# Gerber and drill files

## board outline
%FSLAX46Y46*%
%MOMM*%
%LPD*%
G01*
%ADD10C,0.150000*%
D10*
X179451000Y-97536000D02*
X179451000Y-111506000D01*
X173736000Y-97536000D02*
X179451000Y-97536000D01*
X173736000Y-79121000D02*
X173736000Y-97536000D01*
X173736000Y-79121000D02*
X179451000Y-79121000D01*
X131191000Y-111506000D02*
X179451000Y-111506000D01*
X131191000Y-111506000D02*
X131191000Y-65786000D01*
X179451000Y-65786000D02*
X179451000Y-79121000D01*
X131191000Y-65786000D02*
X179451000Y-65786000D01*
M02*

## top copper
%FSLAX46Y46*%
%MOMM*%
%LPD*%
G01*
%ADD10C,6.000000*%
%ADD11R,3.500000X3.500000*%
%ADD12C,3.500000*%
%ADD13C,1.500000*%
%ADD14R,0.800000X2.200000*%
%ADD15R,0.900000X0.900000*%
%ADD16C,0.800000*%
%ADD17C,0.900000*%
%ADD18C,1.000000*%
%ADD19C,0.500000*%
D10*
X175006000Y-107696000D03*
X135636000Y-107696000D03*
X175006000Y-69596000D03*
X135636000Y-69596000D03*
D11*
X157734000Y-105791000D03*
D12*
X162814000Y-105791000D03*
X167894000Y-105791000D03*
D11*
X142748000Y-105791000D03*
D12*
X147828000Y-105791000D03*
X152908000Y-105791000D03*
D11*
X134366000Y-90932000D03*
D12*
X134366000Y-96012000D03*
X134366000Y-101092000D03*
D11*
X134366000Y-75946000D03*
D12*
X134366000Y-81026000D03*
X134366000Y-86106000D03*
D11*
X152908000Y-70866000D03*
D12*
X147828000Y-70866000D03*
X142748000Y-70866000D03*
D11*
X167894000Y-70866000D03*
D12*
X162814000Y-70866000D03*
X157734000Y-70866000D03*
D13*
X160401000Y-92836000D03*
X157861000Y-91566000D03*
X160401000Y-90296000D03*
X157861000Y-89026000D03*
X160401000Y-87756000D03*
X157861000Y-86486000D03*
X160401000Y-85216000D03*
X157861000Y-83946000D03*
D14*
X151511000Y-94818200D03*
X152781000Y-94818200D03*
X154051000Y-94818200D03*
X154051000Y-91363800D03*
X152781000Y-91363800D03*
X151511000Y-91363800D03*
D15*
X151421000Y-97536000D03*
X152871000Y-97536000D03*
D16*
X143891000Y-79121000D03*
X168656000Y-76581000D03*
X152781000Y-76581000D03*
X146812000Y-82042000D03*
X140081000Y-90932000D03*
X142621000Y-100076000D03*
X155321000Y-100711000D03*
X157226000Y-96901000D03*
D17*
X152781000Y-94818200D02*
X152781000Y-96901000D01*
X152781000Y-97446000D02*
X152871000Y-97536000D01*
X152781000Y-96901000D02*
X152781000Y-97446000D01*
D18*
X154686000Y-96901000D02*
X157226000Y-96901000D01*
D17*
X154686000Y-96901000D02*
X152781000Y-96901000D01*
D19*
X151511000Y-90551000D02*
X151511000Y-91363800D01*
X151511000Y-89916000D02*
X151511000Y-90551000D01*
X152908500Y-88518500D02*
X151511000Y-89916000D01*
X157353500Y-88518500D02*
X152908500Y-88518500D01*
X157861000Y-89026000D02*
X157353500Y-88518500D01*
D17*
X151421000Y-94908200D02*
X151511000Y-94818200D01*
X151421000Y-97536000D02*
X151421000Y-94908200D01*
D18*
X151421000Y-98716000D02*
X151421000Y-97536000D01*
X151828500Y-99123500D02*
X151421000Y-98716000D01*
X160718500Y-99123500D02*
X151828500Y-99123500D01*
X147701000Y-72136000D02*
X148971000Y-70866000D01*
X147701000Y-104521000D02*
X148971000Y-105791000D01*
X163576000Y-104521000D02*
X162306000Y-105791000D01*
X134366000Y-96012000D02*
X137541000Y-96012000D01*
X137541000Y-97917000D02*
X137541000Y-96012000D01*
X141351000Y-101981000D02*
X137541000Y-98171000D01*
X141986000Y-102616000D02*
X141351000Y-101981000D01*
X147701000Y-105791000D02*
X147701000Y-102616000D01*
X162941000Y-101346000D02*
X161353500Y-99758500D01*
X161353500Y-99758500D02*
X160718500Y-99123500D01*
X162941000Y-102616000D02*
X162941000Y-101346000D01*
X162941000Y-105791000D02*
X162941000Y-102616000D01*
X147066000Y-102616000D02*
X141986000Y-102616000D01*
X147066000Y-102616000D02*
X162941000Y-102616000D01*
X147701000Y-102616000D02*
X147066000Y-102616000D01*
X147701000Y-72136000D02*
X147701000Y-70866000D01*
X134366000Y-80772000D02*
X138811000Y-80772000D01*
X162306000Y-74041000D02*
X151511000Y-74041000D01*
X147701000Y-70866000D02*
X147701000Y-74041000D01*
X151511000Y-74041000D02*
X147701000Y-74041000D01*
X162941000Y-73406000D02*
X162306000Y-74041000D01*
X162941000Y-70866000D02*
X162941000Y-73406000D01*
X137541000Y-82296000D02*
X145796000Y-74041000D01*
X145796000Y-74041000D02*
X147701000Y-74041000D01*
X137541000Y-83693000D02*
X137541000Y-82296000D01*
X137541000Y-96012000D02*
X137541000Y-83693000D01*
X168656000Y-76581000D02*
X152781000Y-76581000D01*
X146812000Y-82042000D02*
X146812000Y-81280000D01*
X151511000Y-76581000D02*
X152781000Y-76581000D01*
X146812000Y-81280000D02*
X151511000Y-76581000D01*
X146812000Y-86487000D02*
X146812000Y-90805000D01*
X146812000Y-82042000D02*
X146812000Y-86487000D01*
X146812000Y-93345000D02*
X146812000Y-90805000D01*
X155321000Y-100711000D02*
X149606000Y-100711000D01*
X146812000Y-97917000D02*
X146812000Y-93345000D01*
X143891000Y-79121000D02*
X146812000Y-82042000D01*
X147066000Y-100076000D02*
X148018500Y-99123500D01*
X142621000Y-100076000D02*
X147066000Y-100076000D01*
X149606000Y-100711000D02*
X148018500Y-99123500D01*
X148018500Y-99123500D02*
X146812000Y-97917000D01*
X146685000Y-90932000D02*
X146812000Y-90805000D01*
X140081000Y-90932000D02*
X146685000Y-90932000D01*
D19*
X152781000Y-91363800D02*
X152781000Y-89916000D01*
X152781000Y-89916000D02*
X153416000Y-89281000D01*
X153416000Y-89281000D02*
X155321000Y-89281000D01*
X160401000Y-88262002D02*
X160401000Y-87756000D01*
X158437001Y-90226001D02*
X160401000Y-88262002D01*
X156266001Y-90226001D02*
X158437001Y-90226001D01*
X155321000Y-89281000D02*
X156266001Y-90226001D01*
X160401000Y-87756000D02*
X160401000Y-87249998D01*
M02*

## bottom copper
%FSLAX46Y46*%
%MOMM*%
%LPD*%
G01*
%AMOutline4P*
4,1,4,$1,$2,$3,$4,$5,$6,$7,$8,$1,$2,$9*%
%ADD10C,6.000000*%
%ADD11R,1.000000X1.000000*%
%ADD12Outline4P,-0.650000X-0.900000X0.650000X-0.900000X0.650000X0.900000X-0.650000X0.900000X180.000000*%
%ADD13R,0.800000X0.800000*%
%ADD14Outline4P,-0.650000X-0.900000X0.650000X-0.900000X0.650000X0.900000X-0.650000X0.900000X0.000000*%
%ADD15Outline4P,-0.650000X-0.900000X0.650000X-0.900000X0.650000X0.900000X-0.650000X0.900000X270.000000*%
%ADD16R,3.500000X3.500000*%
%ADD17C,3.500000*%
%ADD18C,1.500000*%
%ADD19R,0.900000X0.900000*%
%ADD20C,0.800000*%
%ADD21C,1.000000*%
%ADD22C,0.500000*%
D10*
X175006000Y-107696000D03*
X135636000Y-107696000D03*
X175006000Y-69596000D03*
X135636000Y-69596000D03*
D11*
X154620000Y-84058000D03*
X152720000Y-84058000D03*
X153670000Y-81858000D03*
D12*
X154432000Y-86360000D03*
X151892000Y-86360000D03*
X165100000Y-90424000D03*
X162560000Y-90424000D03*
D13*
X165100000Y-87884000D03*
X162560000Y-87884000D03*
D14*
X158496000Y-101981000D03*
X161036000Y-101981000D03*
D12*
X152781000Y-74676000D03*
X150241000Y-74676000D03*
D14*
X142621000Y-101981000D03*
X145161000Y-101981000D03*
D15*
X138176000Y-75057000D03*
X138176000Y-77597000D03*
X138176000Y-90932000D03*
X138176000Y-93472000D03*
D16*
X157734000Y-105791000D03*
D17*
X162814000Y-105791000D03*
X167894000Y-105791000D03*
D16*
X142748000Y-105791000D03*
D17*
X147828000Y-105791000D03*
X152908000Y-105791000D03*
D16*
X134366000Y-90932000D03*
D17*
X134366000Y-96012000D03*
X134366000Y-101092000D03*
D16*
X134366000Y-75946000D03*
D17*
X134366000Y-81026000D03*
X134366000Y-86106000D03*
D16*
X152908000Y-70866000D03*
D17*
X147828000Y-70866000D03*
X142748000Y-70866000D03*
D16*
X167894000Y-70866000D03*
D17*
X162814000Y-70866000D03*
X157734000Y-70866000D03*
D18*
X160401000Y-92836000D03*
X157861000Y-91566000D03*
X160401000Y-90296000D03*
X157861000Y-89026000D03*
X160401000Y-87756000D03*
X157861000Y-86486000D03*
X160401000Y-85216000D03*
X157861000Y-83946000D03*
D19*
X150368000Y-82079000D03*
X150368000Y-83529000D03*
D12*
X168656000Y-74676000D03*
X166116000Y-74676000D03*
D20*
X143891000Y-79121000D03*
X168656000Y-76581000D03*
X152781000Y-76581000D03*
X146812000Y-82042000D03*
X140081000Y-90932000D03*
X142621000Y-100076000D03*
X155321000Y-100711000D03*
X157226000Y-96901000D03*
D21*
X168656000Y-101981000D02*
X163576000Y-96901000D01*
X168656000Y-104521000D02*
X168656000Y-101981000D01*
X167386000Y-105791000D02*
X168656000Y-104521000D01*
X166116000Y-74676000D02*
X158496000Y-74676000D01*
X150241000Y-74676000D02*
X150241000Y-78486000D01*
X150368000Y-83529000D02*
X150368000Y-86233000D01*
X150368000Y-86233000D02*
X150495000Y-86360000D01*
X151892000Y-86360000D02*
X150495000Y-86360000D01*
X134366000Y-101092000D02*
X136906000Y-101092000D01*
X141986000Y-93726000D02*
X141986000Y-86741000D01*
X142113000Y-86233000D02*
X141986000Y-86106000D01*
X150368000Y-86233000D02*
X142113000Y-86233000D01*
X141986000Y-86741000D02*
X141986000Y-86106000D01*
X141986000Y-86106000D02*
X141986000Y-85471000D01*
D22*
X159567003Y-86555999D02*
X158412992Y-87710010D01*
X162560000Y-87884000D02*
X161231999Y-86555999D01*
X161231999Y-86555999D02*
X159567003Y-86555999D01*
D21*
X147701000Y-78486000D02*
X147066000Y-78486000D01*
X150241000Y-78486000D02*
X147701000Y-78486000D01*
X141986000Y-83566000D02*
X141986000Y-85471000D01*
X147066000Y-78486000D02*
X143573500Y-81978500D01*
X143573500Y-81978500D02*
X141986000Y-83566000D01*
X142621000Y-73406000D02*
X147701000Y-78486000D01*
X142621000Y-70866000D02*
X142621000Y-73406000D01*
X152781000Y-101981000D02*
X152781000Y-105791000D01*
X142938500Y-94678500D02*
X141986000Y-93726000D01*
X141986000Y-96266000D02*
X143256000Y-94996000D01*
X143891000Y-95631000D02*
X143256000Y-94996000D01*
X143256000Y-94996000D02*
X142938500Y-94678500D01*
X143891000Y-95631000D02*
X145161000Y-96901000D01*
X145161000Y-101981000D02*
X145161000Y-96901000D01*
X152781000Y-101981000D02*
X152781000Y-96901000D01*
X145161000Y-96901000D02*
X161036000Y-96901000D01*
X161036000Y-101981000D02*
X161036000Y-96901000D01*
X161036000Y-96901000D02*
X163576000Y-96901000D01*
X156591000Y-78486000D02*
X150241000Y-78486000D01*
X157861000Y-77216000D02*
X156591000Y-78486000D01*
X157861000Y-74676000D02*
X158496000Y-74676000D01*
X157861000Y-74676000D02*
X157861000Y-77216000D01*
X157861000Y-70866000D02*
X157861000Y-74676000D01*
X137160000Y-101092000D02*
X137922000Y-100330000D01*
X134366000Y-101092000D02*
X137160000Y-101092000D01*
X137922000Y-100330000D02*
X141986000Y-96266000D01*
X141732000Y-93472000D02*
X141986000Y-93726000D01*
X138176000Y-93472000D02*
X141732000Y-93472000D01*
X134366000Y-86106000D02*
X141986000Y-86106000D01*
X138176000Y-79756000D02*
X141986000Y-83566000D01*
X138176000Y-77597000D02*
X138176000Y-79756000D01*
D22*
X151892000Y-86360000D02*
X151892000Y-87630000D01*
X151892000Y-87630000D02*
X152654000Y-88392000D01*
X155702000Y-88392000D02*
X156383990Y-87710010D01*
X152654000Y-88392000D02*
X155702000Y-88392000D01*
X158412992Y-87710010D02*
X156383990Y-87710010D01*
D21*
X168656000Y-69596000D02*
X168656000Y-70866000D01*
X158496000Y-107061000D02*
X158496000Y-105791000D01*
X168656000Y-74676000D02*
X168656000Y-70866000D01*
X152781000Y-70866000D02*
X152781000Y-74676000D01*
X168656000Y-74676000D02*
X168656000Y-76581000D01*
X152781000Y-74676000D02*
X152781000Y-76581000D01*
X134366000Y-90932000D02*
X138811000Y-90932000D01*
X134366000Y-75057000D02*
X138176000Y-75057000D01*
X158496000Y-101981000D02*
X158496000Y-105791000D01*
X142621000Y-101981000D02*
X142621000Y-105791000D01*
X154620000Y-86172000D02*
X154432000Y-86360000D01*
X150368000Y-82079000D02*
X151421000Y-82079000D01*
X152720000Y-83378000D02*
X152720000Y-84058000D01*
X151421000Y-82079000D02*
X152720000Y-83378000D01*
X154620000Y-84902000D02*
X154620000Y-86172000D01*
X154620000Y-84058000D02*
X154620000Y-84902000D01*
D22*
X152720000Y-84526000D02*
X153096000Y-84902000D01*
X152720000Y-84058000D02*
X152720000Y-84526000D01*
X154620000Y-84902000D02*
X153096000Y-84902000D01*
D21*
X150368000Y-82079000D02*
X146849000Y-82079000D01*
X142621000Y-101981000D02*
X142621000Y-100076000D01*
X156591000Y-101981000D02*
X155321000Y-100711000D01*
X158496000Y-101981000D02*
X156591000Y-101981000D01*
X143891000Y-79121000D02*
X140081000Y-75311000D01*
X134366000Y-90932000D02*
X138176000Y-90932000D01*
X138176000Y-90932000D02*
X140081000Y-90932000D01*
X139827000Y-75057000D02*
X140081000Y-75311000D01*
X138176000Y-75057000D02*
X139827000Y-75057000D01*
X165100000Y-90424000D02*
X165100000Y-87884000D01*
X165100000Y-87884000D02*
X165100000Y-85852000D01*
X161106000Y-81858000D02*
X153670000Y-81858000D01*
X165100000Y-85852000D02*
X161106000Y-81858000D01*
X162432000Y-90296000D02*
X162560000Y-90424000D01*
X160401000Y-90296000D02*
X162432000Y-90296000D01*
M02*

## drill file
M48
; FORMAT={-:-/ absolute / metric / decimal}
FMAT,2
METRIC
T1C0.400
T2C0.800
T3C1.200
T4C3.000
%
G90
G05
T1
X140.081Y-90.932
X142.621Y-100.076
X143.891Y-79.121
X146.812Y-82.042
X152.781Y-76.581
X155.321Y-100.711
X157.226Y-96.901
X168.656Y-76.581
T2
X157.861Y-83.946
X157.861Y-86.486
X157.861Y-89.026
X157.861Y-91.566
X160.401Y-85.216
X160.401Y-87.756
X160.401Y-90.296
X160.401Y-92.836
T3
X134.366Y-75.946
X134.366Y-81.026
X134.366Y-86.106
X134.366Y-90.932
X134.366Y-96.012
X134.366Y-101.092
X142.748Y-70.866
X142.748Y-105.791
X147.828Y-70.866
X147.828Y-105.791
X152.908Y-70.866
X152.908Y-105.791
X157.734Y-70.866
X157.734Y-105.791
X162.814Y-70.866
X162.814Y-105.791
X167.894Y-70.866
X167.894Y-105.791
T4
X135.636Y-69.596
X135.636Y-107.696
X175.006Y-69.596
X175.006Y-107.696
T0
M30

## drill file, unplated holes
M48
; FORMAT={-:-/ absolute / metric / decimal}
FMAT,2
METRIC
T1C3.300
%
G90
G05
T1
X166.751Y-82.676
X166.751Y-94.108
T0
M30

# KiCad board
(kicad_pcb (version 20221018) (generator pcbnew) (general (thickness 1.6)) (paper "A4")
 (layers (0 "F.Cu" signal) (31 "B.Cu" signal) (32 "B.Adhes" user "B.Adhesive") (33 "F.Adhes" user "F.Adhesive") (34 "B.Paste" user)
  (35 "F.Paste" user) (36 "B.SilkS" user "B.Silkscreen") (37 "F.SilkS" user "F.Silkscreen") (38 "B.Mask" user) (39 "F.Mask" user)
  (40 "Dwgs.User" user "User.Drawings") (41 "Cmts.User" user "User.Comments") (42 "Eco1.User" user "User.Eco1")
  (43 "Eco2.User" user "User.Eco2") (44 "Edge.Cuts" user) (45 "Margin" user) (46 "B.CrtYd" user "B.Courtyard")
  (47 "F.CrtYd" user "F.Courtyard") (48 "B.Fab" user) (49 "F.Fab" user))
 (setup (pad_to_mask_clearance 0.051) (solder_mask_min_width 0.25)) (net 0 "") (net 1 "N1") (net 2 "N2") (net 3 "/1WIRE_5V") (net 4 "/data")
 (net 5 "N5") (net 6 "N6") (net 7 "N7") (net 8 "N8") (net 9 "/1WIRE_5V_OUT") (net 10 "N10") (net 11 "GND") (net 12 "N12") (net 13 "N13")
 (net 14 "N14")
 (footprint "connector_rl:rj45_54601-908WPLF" (layer "F.Cu") (at 166.751 88.392 90)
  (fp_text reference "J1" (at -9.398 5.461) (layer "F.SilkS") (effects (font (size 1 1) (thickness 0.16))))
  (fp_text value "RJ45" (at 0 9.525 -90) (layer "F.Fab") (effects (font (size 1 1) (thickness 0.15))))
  (pad "" np_thru_hole circle (at -5.716 0 90) (size 3.3 3.3) (drill 3.3) (layers "*.Cu" "*.SilkS" "*.Mask"))
  (pad "" np_thru_hole circle (at 5.716 0 90) (size 3.3 3.3) (drill 3.3) (layers "*.Cu" "*.SilkS" "*.Mask"))
  (pad "1" thru_hole circle (at -4.444 -6.35 90) (size 1.5 1.5) (drill 0.8) (layers "*.Cu" "*.Mask") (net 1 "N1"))
  (pad "2" thru_hole circle (at -3.174 -8.89 90) (size 1.5 1.5) (drill 0.8) (layers "*.Cu" "*.Mask") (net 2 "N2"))
  (pad "3" thru_hole circle (at -1.904 -6.35 90) (size 1.5 1.5) (drill 0.8) (layers "*.Cu" "*.Mask") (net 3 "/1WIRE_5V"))
  (pad "4" thru_hole circle (at -0.634 -8.89 90) (size 1.5 1.5) (drill 0.8) (layers "*.Cu" "*.Mask") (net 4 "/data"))
  (pad "5" thru_hole circle (at 0.636 -6.35 90) (size 1.5 1.5) (drill 0.8) (layers "*.Cu" "*.Mask") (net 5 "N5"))
  (pad "6" thru_hole circle (at 1.906 -8.89 270) (size 1.5 1.5) (drill 0.8) (layers "*.Cu" "*.Mask") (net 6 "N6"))
  (pad "7" thru_hole circle (at 3.176 -6.35 90) (size 1.5 1.5) (drill 0.8) (layers "*.Cu" "*.Mask") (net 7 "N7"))
  (pad "8" thru_hole circle (at 4.446 -8.89 90) (size 1.5 1.5) (drill 0.8) (layers "*.Cu" "*.Mask") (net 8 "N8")))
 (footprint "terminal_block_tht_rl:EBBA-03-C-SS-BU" (layer "F.Cu") (at 162.814 70.866 180)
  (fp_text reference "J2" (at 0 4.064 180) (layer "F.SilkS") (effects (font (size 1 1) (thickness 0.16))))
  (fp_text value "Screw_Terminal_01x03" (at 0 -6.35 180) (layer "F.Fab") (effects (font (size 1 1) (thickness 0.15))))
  (pad "1" thru_hole rect (at -5.08 0) (size 3.5 3.5) (drill 1.2) (layers "*.Cu" "*.Mask") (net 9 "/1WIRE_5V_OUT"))
  (pad "2" thru_hole circle (at 0 0) (size 3.5 3.5) (drill 1.2) (layers "*.Cu" "*.Mask") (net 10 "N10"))
  (pad "3" thru_hole circle (at 5.08 0) (size 3.5 3.5) (drill 1.2) (layers "*.Cu" "*.Mask") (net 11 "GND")))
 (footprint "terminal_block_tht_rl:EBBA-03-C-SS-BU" (layer "F.Cu") (at 134.366 81.026 -90)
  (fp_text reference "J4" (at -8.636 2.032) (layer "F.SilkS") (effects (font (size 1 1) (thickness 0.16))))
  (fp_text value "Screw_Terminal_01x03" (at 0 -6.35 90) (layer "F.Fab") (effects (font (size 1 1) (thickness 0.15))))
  (pad "1" thru_hole rect (at -5.08 0 90) (size 3.5 3.5) (drill 1.2) (layers "*.Cu" "*.Mask") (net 9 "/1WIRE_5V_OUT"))
  (pad "2" thru_hole circle (at 0 0 90) (size 3.5 3.5) (drill 1.2) (layers "*.Cu" "*.Mask") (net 10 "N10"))
  (pad "3" thru_hole circle (at 5.08 0 90) (size 3.5 3.5) (drill 1.2) (layers "*.Cu" "*.Mask") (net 11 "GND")))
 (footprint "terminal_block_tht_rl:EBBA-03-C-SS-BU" (layer "F.Cu") (at 134.366 96.012 -90)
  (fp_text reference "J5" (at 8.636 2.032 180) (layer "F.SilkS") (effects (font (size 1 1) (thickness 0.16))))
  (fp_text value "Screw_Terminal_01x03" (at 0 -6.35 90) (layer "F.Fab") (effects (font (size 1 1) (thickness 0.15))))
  (pad "1" thru_hole rect (at -5.08 0 90) (size 3.5 3.5) (drill 1.2) (layers "*.Cu" "*.Mask") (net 9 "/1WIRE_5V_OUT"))
  (pad "2" thru_hole circle (at 0 0 90) (size 3.5 3.5) (drill 1.2) (layers "*.Cu" "*.Mask") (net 10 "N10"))
  (pad "3" thru_hole circle (at 5.08 0 90) (size 3.5 3.5) (drill 1.2) (layers "*.Cu" "*.Mask") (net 11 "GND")))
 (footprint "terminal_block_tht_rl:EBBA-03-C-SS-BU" (layer "F.Cu") (at 147.828 70.866 180)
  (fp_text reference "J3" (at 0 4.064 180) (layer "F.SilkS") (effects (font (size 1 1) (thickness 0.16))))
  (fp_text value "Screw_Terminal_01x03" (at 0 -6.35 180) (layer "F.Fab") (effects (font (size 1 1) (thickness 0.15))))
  (pad "1" thru_hole rect (at -5.08 0) (size 3.5 3.5) (drill 1.2) (layers "*.Cu" "*.Mask") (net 9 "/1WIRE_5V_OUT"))
  (pad "2" thru_hole circle (at 0 0) (size 3.5 3.5) (drill 1.2) (layers "*.Cu" "*.Mask") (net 10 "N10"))
  (pad "3" thru_hole circle (at 5.08 0) (size 3.5 3.5) (drill 1.2) (layers "*.Cu" "*.Mask") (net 11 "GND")))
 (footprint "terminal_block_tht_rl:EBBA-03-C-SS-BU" (layer "F.Cu") (at 147.828 105.791)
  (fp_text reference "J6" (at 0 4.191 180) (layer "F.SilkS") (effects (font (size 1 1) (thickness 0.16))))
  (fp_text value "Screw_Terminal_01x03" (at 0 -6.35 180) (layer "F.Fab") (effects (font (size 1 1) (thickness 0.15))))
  (pad "1" thru_hole rect (at -5.08 0 180) (size 3.5 3.5) (drill 1.2) (layers "*.Cu" "*.Mask") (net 9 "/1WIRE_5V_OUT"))
  (pad "2" thru_hole circle (at 0 0 180) (size 3.5 3.5) (drill 1.2) (layers "*.Cu" "*.Mask") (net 10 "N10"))
  (pad "3" thru_hole circle (at 5.08 0 180) (size 3.5 3.5) (drill 1.2) (layers "*.Cu" "*.Mask") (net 11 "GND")))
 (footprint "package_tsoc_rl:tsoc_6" (layer "F.Cu") (at 152.781 93.091 90)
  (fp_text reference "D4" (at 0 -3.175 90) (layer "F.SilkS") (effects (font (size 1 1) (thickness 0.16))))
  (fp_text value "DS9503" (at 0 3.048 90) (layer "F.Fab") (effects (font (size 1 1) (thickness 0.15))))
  (pad "1" smd rect (at -1.7272 -1.27 90) (size 2.2 0.8) (layers "F.Cu" "F.Paste" "F.Mask") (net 10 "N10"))
  (pad "2" smd rect (at -1.7272 0 90) (size 2.2 0.8) (layers "F.Cu" "F.Paste" "F.Mask") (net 11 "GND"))
  (pad "3" smd rect (at -1.7272 1.27 90) (size 2.2 0.8) (layers "F.Cu" "F.Paste" "F.Mask") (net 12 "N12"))
  (pad "4" smd rect (at 1.7272 1.27 90) (size 2.2 0.8) (layers "F.Cu" "F.Paste" "F.Mask") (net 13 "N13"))
  (pad "5" smd rect (at 1.7272 0 90) (size 2.2 0.8) (layers "F.Cu" "F.Paste" "F.Mask") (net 5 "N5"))
  (pad "6" smd rect (at 1.7272 -1.27 90) (size 2.2 0.8) (layers "F.Cu" "F.Paste" "F.Mask") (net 4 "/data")))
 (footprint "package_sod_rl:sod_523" (layer "F.Cu") (at 152.146 97.536)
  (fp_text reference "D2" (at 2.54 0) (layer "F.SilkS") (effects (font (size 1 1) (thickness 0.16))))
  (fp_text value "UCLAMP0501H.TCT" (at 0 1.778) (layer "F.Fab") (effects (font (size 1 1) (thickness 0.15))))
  (pad "1" smd rect (at -0.725 0) (size 0.9 0.9) (layers "F.Cu" "F.Paste" "F.Mask") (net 10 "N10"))
  (pad "2" smd rect (at 0.725 0) (size 0.9 0.9) (layers "F.Cu" "F.Paste" "F.Mask") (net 11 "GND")))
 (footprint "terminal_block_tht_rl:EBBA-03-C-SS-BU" (layer "F.Cu") (at 162.814 105.791)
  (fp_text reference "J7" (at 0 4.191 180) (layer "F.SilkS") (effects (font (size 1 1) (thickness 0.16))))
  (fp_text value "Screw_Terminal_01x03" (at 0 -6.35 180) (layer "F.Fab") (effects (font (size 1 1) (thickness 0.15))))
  (pad "1" thru_hole rect (at -5.08 0 180) (size 3.5 3.5) (drill 1.2) (layers "*.Cu" "*.Mask") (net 9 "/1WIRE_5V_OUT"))
  (pad "2" thru_hole circle (at 0 0 180) (size 3.5 3.5) (drill 1.2) (layers "*.Cu" "*.Mask") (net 10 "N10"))
  (pad "3" thru_hole circle (at 5.08 0 180) (size 3.5 3.5) (drill 1.2) (layers "*.Cu" "*.Mask") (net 11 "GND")))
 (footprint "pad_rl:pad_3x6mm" (layer "F.Cu") (at 135.636 69.596)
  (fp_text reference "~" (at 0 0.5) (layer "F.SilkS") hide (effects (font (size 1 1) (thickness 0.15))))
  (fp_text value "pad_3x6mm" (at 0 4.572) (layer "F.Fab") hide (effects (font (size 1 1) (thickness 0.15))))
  (pad "~" thru_hole circle (at 0 0) (size 6 6) (drill 3) (layers "*.Cu" "*.Mask")))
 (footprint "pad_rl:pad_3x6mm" (layer "F.Cu") (at 175.006 69.596)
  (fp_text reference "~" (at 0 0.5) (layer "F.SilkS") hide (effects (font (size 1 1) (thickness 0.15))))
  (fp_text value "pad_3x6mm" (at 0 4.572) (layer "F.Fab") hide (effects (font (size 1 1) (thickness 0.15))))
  (pad "~" thru_hole circle (at 0 0) (size 6 6) (drill 3) (layers "*.Cu" "*.Mask")))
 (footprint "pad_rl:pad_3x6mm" (layer "F.Cu") (at 135.636 107.696)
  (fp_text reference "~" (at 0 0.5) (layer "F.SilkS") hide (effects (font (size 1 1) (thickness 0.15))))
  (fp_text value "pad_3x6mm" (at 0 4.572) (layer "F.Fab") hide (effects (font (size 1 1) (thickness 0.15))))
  (pad "~" thru_hole circle (at 0 0) (size 6 6) (drill 3) (layers "*.Cu" "*.Mask")))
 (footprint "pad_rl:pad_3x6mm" (layer "F.Cu") (at 175.006 107.696)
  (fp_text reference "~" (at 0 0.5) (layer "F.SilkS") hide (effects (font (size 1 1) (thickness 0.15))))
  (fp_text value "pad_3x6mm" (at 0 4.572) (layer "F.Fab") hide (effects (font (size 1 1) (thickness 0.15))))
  (pad "~" thru_hole circle (at 0 0) (size 6 6) (drill 3) (layers "*.Cu" "*.Mask")))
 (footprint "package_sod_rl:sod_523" (layer "B.Cu") (at 150.368 82.804 -90)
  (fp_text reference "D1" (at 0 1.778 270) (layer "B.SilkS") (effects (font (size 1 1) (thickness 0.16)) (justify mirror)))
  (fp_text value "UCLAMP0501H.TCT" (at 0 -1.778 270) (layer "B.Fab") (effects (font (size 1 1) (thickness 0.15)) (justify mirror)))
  (pad "1" smd rect (at -0.725 0 270) (size 0.9 0.9) (layers "B.Cu" "B.Paste" "B.Mask") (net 9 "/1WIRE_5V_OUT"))
  (pad "2" smd rect (at 0.725 0 270) (size 0.9 0.9) (layers "B.Cu" "B.Paste" "B.Mask") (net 11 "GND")))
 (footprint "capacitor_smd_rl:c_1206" (layer "B.Cu") (at 167.386 74.676 180)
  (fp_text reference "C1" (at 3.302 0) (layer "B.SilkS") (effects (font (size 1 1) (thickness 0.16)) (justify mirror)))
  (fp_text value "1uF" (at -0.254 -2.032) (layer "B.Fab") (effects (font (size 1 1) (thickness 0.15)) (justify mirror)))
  (pad "1" smd trapezoid (at -1.27 0 180) (size 1.3 1.8) (layers "B.Cu" "B.Paste" "B.Mask") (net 9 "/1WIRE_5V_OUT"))
  (pad "2" smd trapezoid (at 1.27 0 180) (size 1.3 1.8) (layers "B.Cu" "B.Paste" "B.Mask") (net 11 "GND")))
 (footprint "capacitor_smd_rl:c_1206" (layer "B.Cu") (at 138.176 92.202 -90)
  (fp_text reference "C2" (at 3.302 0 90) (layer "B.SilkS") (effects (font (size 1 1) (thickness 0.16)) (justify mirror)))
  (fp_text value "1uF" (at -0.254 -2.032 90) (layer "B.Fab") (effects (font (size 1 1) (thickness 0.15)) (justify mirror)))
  (pad "1" smd trapezoid (at -1.27 0 270) (size 1.3 1.8) (layers "B.Cu" "B.Paste" "B.Mask") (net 9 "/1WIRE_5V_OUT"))
  (pad "2" smd trapezoid (at 1.27 0 270) (size 1.3 1.8) (layers "B.Cu" "B.Paste" "B.Mask") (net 11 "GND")))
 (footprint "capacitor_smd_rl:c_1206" (layer "B.Cu") (at 151.511 74.676 180)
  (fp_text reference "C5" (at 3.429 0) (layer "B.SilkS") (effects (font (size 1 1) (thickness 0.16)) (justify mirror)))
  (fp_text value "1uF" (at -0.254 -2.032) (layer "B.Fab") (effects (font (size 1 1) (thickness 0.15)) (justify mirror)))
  (pad "1" smd trapezoid (at -1.27 0 180) (size 1.3 1.8) (layers "B.Cu" "B.Paste" "B.Mask") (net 9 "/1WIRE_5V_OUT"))
  (pad "2" smd trapezoid (at 1.27 0 180) (size 1.3 1.8) (layers "B.Cu" "B.Paste" "B.Mask") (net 11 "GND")))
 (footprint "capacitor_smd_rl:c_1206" (layer "B.Cu") (at 143.891 101.981)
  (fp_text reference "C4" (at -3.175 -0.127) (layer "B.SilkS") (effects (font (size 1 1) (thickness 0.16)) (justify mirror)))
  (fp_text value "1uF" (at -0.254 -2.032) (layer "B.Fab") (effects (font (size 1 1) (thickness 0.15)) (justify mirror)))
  (pad "1" smd trapezoid (at -1.27 0) (size 1.3 1.8) (layers "B.Cu" "B.Paste" "B.Mask") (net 9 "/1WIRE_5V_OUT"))
  (pad "2" smd trapezoid (at 1.27 0) (size 1.3 1.8) (layers "B.Cu" "B.Paste" "B.Mask") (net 11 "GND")))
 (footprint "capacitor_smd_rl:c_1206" (layer "B.Cu") (at 159.766 101.981)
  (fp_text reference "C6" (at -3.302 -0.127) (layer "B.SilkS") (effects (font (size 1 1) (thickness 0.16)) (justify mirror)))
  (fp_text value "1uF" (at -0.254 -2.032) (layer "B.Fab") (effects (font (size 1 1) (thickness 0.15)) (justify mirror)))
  (pad "1" smd trapezoid (at -1.27 0) (size 1.3 1.8) (layers "B.Cu" "B.Paste" "B.Mask") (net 9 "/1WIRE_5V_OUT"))
  (pad "2" smd trapezoid (at 1.27 0) (size 1.3 1.8) (layers "B.Cu" "B.Paste" "B.Mask") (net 11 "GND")))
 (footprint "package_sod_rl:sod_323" (layer "B.Cu") (at 163.83 87.884 180)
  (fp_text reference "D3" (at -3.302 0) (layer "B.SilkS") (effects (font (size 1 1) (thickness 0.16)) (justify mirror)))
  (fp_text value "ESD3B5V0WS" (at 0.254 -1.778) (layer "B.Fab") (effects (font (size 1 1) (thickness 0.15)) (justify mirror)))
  (pad "1" smd rect (at -1.27 0 180) (size 0.8 0.8) (layers "B.Cu" "B.Paste" "B.Mask") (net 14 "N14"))
  (pad "2" smd rect (at 1.27 0 180) (size 0.8 0.8) (layers "B.Cu" "B.Paste" "B.Mask") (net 11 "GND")))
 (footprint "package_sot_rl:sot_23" (layer "B.Cu") (at 153.67 83.058 90)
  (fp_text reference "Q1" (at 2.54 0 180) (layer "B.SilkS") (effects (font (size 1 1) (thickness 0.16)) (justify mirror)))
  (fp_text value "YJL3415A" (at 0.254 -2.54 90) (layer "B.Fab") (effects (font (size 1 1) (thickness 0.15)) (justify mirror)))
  (pad "1" smd rect (at -1 0.95 90) (size 1 1) (layers "B.Cu" "B.Paste" "B.Mask") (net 9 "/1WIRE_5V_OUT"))
  (pad "2" smd rect (at -1 -0.95 90) (size 1 1) (layers "B.Cu" "B.Paste" "B.Mask") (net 9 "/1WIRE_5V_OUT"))
  (pad "3" smd rect (at 1.2 0 90) (size 1 1) (layers "B.Cu" "B.Paste" "B.Mask") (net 14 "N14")))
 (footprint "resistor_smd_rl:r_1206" (layer "B.Cu") (at 163.83 90.424 180)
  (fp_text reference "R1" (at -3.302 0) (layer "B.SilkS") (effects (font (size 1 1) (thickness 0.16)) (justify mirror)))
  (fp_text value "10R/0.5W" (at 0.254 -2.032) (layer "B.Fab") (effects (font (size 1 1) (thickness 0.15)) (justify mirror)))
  (pad "1" smd trapezoid (at -1.27 0 180) (size 1.3 1.8) (layers "B.Cu" "B.Paste" "B.Mask") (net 14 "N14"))
  (pad "2" smd trapezoid (at 1.27 0 180) (size 1.3 1.8) (layers "B.Cu" "B.Paste" "B.Mask") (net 3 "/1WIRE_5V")))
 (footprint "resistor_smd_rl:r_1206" (layer "B.Cu") (at 153.162 86.36 180)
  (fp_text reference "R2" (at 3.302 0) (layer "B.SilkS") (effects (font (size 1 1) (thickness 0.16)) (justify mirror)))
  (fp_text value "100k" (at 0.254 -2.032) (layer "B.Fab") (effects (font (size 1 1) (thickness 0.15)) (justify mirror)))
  (pad "1" smd trapezoid (at -1.27 0 180) (size 1.3 1.8) (layers "B.Cu" "B.Paste" "B.Mask") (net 9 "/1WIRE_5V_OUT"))
  (pad "2" smd trapezoid (at 1.27 0 180) (size 1.3 1.8) (layers "B.Cu" "B.Paste" "B.Mask") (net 11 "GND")))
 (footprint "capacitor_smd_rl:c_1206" (layer "B.Cu") (at 138.176 76.327 -90)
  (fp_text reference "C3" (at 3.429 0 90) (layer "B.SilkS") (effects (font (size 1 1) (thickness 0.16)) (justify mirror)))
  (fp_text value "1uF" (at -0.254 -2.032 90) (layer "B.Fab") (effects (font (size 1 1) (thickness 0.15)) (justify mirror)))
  (pad "1" smd trapezoid (at -1.27 0 270) (size 1.3 1.8) (layers "B.Cu" "B.Paste" "B.Mask") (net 9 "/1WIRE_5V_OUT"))
  (pad "2" smd trapezoid (at 1.27 0 270) (size 1.3 1.8) (layers "B.Cu" "B.Paste" "B.Mask") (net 11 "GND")))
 (gr_line (start 131.191 111.506) (end 131.191 65.786) (stroke (width 0.15) (type solid)) (layer "Edge.Cuts"))
 (gr_line (start 179.451 65.786) (end 179.451 79.121) (stroke (width 0.15) (type solid)) (layer "Edge.Cuts"))
 (gr_line (start 131.191 111.506) (end 179.451 111.506) (stroke (width 0.15) (type solid)) (layer "Edge.Cuts"))
 (gr_line (start 173.736 79.121) (end 179.451 79.121) (stroke (width 0.15) (type solid)) (layer "Edge.Cuts"))
 (gr_line (start 173.736 79.121) (end 173.736 97.536) (stroke (width 0.15) (type solid)) (layer "Edge.Cuts"))
 (gr_line (start 173.736 97.536) (end 179.451 97.536) (stroke (width 0.15) (type solid)) (layer "Edge.Cuts"))
 (gr_line (start 179.451 97.536) (end 179.451 111.506) (stroke (width 0.15) (type solid)) (layer "Edge.Cuts"))
 (gr_line (start 131.191 65.786) (end 179.451 65.786) (stroke (width 0.15) (type solid)) (layer "Edge.Cuts"))
 (segment (start 152.781 94.8182) (end 152.781 96.901) (width 0.9) (layer "F.Cu") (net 11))
 (segment (start 154.686 96.901) (end 157.226 96.901) (width 1) (layer "F.Cu") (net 11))
 (segment (start 152.781 97.446) (end 152.871 97.536) (width 0.9) (layer "F.Cu") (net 11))
 (segment (start 154.686 96.901) (end 152.781 96.901) (width 0.9) (layer "F.Cu") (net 11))
 (segment (start 152.781 96.901) (end 152.781 97.446) (width 0.9) (layer "F.Cu") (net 11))
 (via (at 157.226 96.901) (size 0.8) (drill 0.4) (layers "F.Cu" "B.Cu") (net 11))
 (segment (start 141.986 83.566) (end 141.986 85.471) (width 1) (layer "B.Cu") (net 11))
 (segment (start 142.621 73.406) (end 147.701 78.486) (width 1) (layer "B.Cu") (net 11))
 (segment (start 138.176 79.756) (end 141.986 83.566) (width 1) (layer "B.Cu") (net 11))
 (segment (start 141.986 93.726) (end 141.986 86.741) (width 1) (layer "B.Cu") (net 11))
 (segment (start 150.241 74.676) (end 150.241 78.486) (width 1) (layer "B.Cu") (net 11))
 (segment (start 151.892 86.36) (end 150.495 86.36) (width 1) (layer "B.Cu") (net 11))
 (segment (start 137.922 100.33) (end 141.986 96.266) (width 1) (layer "B.Cu") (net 11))
 (segment (start 150.368 86.233) (end 150.495 86.36) (width 1) (layer "B.Cu") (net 11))
 (segment (start 168.656 104.521) (end 168.656 101.981) (width 1) (layer "B.Cu") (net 11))
 (segment (start 143.891 95.631) (end 143.256 94.996) (width 1) (layer "B.Cu") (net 11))
 (segment (start 137.16 101.092) (end 137.922 100.33) (width 1) (layer "B.Cu") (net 11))
 (segment (start 134.366 86.106) (end 141.986 86.106) (width 1) (layer "B.Cu") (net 11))
 (segment (start 141.732 93.472) (end 141.986 93.726) (width 1) (layer "B.Cu") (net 11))
 (segment (start 167.386 105.791) (end 168.656 104.521) (width 1) (layer "B.Cu") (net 11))
 (segment (start 155.702 88.392) (end 156.38399 87.71001) (width 0.5) (layer "B.Cu") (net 11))
 (segment (start 147.701 78.486) (end 147.066 78.486) (width 1) (layer "B.Cu") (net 11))
 (segment (start 161.036 101.981) (end 161.036 96.901) (width 1) (layer "B.Cu") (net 11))
 (segment (start 168.656 101.981) (end 163.576 96.901) (width 1) (layer "B.Cu") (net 11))
 (segment (start 150.368 83.529) (end 150.368 86.233) (width 1) (layer "B.Cu") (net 11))
 (segment (start 158.412992 87.71001) (end 156.38399 87.71001) (width 0.5) (layer "B.Cu") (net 11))
 (segment (start 145.161 96.901) (end 161.036 96.901) (width 1) (layer "B.Cu") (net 11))
 (segment (start 145.161 101.981) (end 145.161 96.901) (width 1) (layer "B.Cu") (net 11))
 (segment (start 161.231999 86.555999) (end 159.567003 86.555999) (width 0.5) (layer "B.Cu") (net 11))
 (segment (start 159.567003 86.555999) (end 158.412992 87.71001) (width 0.5) (layer "B.Cu") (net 11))
 (segment (start 152.781 101.981) (end 152.781 105.791) (width 1) (layer "B.Cu") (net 11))
 (segment (start 150.368 86.233) (end 142.113 86.233) (width 1) (layer "B.Cu") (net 11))
 (segment (start 166.116 74.676) (end 158.496 74.676) (width 1) (layer "B.Cu") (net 11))
 (segment (start 152.654 88.392) (end 155.702 88.392) (width 0.5) (layer "B.Cu") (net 11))
 (segment (start 142.9385 94.6785) (end 141.986 93.726) (width 1) (layer "B.Cu") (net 11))
 (segment (start 162.56 87.884) (end 161.231999 86.555999) (width 0.5) (layer "B.Cu") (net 11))
 (segment (start 138.176 93.472) (end 141.732 93.472) (width 1) (layer "B.Cu") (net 11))
 (segment (start 152.781 101.981) (end 152.781 96.901) (width 1) (layer "B.Cu") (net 11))
 (segment (start 143.891 95.631) (end 145.161 96.901) (width 1) (layer "B.Cu") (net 11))
 (segment (start 143.256 94.996) (end 142.9385 94.6785) (width 1) (layer "B.Cu") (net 11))
 (segment (start 151.892 87.63) (end 152.654 88.392) (width 0.5) (layer "B.Cu") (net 11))
 (segment (start 142.113 86.233) (end 141.986 86.106) (width 1) (layer "B.Cu") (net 11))
 (segment (start 151.892 86.36) (end 151.892 87.63) (width 0.5) (layer "B.Cu") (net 11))
 (segment (start 134.366 101.092) (end 136.906 101.092) (width 1) (layer "B.Cu") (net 11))
 (segment (start 157.861 74.676) (end 157.861 77.216) (width 1) (layer "B.Cu") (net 11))
 (segment (start 143.5735 81.9785) (end 141.986 83.566) (width 1) (layer "B.Cu") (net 11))
 (segment (start 142.621 70.866) (end 142.621 73.406) (width 1) (layer "B.Cu") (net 11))
 (segment (start 157.861 74.676) (end 158.496 74.676) (width 1) (layer "B.Cu") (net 11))
 (segment (start 134.366 101.092) (end 137.16 101.092) (width 1) (layer "B.Cu") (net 11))
 (segment (start 147.066 78.486) (end 143.5735 81.9785) (width 1) (layer "B.Cu") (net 11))
 (segment (start 138.176 77.597) (end 138.176 79.756) (width 1) (layer "B.Cu") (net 11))
 (segment (start 141.986 96.266) (end 143.256 94.996) (width 1) (layer "B.Cu") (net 11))
 (segment (start 157.861 77.216) (end 156.591 78.486) (width 1) (layer "B.Cu") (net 11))
 (segment (start 156.591 78.486) (end 150.241 78.486) (width 1) (layer "B.Cu") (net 11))
 (segment (start 150.241 78.486) (end 147.701 78.486) (width 1) (layer "B.Cu") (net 11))
 (segment (start 161.036 96.901) (end 163.576 96.901) (width 1) (layer "B.Cu") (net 11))
 (segment (start 157.861 70.866) (end 157.861 74.676) (width 1) (layer "B.Cu") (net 11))
 (segment (start 141.986 86.106) (end 141.986 85.471) (width 1) (layer "B.Cu") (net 11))
 (segment (start 141.986 86.741) (end 141.986 86.106) (width 1) (layer "B.Cu") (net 11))
 (segment (start 152.9085 88.5185) (end 151.511 89.916) (width 0.5) (layer "F.Cu") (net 4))
 (segment (start 151.511 89.916) (end 151.511 90.551) (width 0.5) (layer "F.Cu") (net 4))
 (segment (start 151.511 90.551) (end 151.511 91.3638) (width 0.5) (layer "F.Cu") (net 4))
 (segment (start 157.3535 88.5185) (end 152.9085 88.5185) (width 0.5) (layer "F.Cu") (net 4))
 (segment (start 157.861 89.026) (end 157.3535 88.5185) (width 0.5) (layer "F.Cu") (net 4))
 (segment (start 134.366 96.012) (end 137.541 96.012) (width 1) (layer "F.Cu") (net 10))
 (segment (start 137.541 96.012) (end 137.541 83.693) (width 1) (layer "F.Cu") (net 10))
 (segment (start 141.351 101.981) (end 137.541 98.171) (width 1) (layer "F.Cu") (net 10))
 (segment (start 162.941 101.346) (end 161.3535 99.7585) (width 1) (layer "F.Cu") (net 10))
 (segment (start 162.941 105.791) (end 162.941 102.616) (width 1) (layer "F.Cu") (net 10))
 (segment (start 162.941 70.866) (end 162.941 73.406) (width 1) (layer "F.Cu") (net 10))
 (segment (start 163.576 104.521) (end 162.306 105.791) (width 1) (layer "F.Cu") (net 10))
 (segment (start 147.701 70.866) (end 147.701 74.041) (width 1) (layer "F.Cu") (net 10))
 (segment (start 137.541 83.693) (end 137.541 82.296) (width 1) (layer "F.Cu") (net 10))
 (segment (start 147.701 72.136) (end 147.701 70.866) (width 1) (layer "F.Cu") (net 10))
 (segment (start 147.701 105.791) (end 147.701 102.616) (width 1) (layer "F.Cu") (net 10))
 (segment (start 151.511 74.041) (end 147.701 74.041) (width 1) (layer "F.Cu") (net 10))
 (segment (start 162.306 74.041) (end 151.511 74.041) (width 1) (layer "F.Cu") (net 10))
 (segment (start 147.701 104.521) (end 148.971 105.791) (width 1) (layer "F.Cu") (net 10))
 (segment (start 147.066 102.616) (end 141.986 102.616) (width 1) (layer "F.Cu") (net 10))
 (segment (start 137.541 97.917) (end 137.541 96.012) (width 1) (layer "F.Cu") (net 10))
 (segment (start 161.3535 99.7585) (end 160.7185 99.1235) (width 1) (layer "F.Cu") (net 10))
 (segment (start 137.541 82.296) (end 145.796 74.041) (width 1) (layer "F.Cu") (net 10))
 (segment (start 145.796 74.041) (end 147.701 74.041) (width 1) (layer "F.Cu") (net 10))
 (segment (start 151.8285 99.1235) (end 151.421 98.716) (width 1) (layer "F.Cu") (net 10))
 (segment (start 160.7185 99.1235) (end 151.8285 99.1235) (width 1) (layer "F.Cu") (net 10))
 (segment (start 151.421 97.536) (end 151.421 94.9082) (width 0.9) (layer "F.Cu") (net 10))
 (segment (start 147.701 102.616) (end 147.066 102.616) (width 1) (layer "F.Cu") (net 10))
 (segment (start 141.986 102.616) (end 141.351 101.981) (width 1) (layer "F.Cu") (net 10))
 (segment (start 147.701 72.136) (end 148.971 70.866) (width 1) (layer "F.Cu") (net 10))
 (segment (start 162.941 73.406) (end 162.306 74.041) (width 1) (layer "F.Cu") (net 10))
 (segment (start 147.066 102.616) (end 162.941 102.616) (width 1) (layer "F.Cu") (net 10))
 (segment (start 151.421 98.716) (end 151.421 97.536) (width 1) (layer "F.Cu") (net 10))
 (segment (start 134.366 80.772) (end 138.811 80.772) (width 1) (layer "F.Cu") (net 10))
 (segment (start 162.941 102.616) (end 162.941 101.346) (width 1) (layer "F.Cu") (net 10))
 (segment (start 151.421 94.9082) (end 151.511 94.8182) (width 0.9) (layer "F.Cu") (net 10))
 (segment (start 142.621 100.076) (end 147.066 100.076) (width 1) (layer "F.Cu") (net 9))
 (segment (start 143.891 79.121) (end 146.812 82.042) (width 1) (layer "F.Cu") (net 9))
 (segment (start 146.812 86.487) (end 146.812 90.805) (width 1) (layer "F.Cu") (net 9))
 (segment (start 151.511 76.581) (end 152.781 76.581) (width 1) (layer "F.Cu") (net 9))
 (segment (start 147.066 100.076) (end 148.0185 99.1235) (width 1) (layer "F.Cu") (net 9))
 (segment (start 146.812 97.917) (end 146.812 93.345) (width 1) (layer "F.Cu") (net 9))
 (segment (start 146.812 93.345) (end 146.812 90.805) (width 1) (layer "F.Cu") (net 9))
 (segment (start 146.812 82.042) (end 146.812 86.487) (width 1) (layer "F.Cu") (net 9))
 (segment (start 140.081 90.932) (end 146.685 90.932) (width 1) (layer "F.Cu") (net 9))
 (segment (start 155.321 100.711) (end 149.606 100.711) (width 1) (layer "F.Cu") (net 9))
 (segment (start 146.812 82.042) (end 146.812 81.28) (width 1) (layer "F.Cu") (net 9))
 (segment (start 168.656 76.581) (end 152.781 76.581) (width 1) (layer "F.Cu") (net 9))
 (segment (start 146.685 90.932) (end 146.812 90.805) (width 1) (layer "F.Cu") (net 9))
 (segment (start 149.606 100.711) (end 148.0185 99.1235) (width 1) (layer "F.Cu") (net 9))
 (segment (start 146.812 81.28) (end 151.511 76.581) (width 1) (layer "F.Cu") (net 9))
 (segment (start 148.0185 99.1235) (end 146.812 97.917) (width 1) (layer "F.Cu") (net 9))
 (via (at 140.081 90.932) (size 0.8) (drill 0.4) (layers "F.Cu" "B.Cu") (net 9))
 (via (at 152.781 76.581) (size 0.8) (drill 0.4) (layers "F.Cu" "B.Cu") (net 9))
 (via (at 168.656 76.581) (size 0.8) (drill 0.4) (layers "F.Cu" "B.Cu") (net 9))
 (via (at 146.812 82.042) (size 0.8) (drill 0.4) (layers "F.Cu" "B.Cu") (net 9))
 (via (at 143.891 79.121) (size 0.8) (drill 0.4) (layers "F.Cu" "B.Cu") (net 9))
 (via (at 155.321 100.711) (size 0.8) (drill 0.4) (layers "F.Cu" "B.Cu") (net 9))
 (via (at 142.621 100.076) (size 0.8) (drill 0.4) (layers "F.Cu" "B.Cu") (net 9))
 (segment (start 154.62 86.172) (end 154.432 86.36) (width 1) (layer "B.Cu") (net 9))
 (segment (start 134.366 90.932) (end 138.811 90.932) (width 1) (layer "B.Cu") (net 9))
 (segment (start 154.62 84.058) (end 154.62 84.902) (width 1) (layer "B.Cu") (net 9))
 (segment (start 139.827 75.057) (end 140.081 75.311) (width 1) (layer "B.Cu") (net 9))
 (segment (start 158.496 101.981) (end 158.496 105.791) (width 1) (layer "B.Cu") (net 9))
 (segment (start 134.366 75.057) (end 138.176 75.057) (width 1) (layer "B.Cu") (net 9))
 (segment (start 152.781 74.676) (end 152.781 76.581) (width 1) (layer "B.Cu") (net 9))
 (segment (start 143.891 79.121) (end 140.081 75.311) (width 1) (layer "B.Cu") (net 9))
 (segment (start 156.591 101.981) (end 155.321 100.711) (width 1) (layer "B.Cu") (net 9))
 (segment (start 168.656 74.676) (end 168.656 70.866) (width 1) (layer "B.Cu") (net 9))
 (segment (start 152.72 83.378) (end 152.72 84.058) (width 1) (layer "B.Cu") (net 9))
 (segment (start 154.62 84.902) (end 153.096 84.902) (width 0.5) (layer "B.Cu") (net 9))
 (segment (start 168.656 74.676) (end 168.656 76.581) (width 1) (layer "B.Cu") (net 9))
 (segment (start 158.496 101.981) (end 156.591 101.981) (width 1) (layer "B.Cu") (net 9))
 (segment (start 152.72 84.526) (end 153.096 84.902) (width 0.5) (layer "B.Cu") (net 9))
 (segment (start 158.496 107.061) (end 158.496 105.791) (width 1) (layer "B.Cu") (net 9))
 (segment (start 138.176 75.057) (end 139.827 75.057) (width 1) (layer "B.Cu") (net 9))
 (segment (start 142.621 101.981) (end 142.621 100.076) (width 1) (layer "B.Cu") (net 9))
 (segment (start 138.176 90.932) (end 140.081 90.932) (width 1) (layer "B.Cu") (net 9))
 (segment (start 150.368 82.079) (end 151.421 82.079) (width 1) (layer "B.Cu") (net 9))
 (segment (start 150.368 82.079) (end 146.849 82.079) (width 1) (layer "B.Cu") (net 9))
 (segment (start 151.421 82.079) (end 152.72 83.378) (width 1) (layer "B.Cu") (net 9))
 (segment (start 168.656 69.596) (end 168.656 70.866) (width 1) (layer "B.Cu") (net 9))
 (segment (start 154.62 84.902) (end 154.62 86.172) (width 1) (layer "B.Cu") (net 9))
 (segment (start 152.72 84.058) (end 152.72 84.526) (width 0.5) (layer "B.Cu") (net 9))
 (segment (start 152.781 70.866) (end 152.781 74.676) (width 1) (layer "B.Cu") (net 9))
 (segment (start 142.621 101.981) (end 142.621 105.791) (width 1) (layer "B.Cu") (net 9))
 (segment (start 134.366 90.932) (end 138.176 90.932) (width 1) (layer "B.Cu") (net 9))
 (segment (start 165.1 85.852) (end 161.106 81.858) (width 1) (layer "B.Cu") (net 14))
 (segment (start 165.1 87.884) (end 165.1 85.852) (width 1) (layer "B.Cu") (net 14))
 (segment (start 165.1 90.424) (end 165.1 87.884) (width 1) (layer "B.Cu") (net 14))
 (segment (start 161.106 81.858) (end 153.67 81.858) (width 1) (layer "B.Cu") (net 14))
 (segment (start 162.432 90.296) (end 162.56 90.424) (width 1) (layer "B.Cu") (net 3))
 (segment (start 160.401 90.296) (end 162.432 90.296) (width 1) (layer "B.Cu") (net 3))
 (segment (start 152.781 91.3638) (end 152.781 89.916) (width 0.5) (layer "F.Cu") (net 5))
 (segment (start 156.266001 90.226001) (end 158.437001 90.226001) (width 0.5) (layer "F.Cu") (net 5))
 (segment (start 158.437001 90.226001) (end 160.401 88.262002) (width 0.5) (layer "F.Cu") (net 5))
 (segment (start 160.401 88.262002) (end 160.401 87.756) (width 0.5) (layer "F.Cu") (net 5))
 (segment (start 152.781 89.916) (end 153.416 89.281) (width 0.5) (layer "F.Cu") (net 5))
 (segment (start 155.321 89.281) (end 156.266001 90.226001) (width 0.5) (layer "F.Cu") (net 5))
 (segment (start 160.401 87.756) (end 160.401 87.249998) (width 0.5) (layer "F.Cu") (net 5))
 (segment (start 153.416 89.281) (end 155.321 89.281) (width 0.5) (layer "F.Cu") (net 5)))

